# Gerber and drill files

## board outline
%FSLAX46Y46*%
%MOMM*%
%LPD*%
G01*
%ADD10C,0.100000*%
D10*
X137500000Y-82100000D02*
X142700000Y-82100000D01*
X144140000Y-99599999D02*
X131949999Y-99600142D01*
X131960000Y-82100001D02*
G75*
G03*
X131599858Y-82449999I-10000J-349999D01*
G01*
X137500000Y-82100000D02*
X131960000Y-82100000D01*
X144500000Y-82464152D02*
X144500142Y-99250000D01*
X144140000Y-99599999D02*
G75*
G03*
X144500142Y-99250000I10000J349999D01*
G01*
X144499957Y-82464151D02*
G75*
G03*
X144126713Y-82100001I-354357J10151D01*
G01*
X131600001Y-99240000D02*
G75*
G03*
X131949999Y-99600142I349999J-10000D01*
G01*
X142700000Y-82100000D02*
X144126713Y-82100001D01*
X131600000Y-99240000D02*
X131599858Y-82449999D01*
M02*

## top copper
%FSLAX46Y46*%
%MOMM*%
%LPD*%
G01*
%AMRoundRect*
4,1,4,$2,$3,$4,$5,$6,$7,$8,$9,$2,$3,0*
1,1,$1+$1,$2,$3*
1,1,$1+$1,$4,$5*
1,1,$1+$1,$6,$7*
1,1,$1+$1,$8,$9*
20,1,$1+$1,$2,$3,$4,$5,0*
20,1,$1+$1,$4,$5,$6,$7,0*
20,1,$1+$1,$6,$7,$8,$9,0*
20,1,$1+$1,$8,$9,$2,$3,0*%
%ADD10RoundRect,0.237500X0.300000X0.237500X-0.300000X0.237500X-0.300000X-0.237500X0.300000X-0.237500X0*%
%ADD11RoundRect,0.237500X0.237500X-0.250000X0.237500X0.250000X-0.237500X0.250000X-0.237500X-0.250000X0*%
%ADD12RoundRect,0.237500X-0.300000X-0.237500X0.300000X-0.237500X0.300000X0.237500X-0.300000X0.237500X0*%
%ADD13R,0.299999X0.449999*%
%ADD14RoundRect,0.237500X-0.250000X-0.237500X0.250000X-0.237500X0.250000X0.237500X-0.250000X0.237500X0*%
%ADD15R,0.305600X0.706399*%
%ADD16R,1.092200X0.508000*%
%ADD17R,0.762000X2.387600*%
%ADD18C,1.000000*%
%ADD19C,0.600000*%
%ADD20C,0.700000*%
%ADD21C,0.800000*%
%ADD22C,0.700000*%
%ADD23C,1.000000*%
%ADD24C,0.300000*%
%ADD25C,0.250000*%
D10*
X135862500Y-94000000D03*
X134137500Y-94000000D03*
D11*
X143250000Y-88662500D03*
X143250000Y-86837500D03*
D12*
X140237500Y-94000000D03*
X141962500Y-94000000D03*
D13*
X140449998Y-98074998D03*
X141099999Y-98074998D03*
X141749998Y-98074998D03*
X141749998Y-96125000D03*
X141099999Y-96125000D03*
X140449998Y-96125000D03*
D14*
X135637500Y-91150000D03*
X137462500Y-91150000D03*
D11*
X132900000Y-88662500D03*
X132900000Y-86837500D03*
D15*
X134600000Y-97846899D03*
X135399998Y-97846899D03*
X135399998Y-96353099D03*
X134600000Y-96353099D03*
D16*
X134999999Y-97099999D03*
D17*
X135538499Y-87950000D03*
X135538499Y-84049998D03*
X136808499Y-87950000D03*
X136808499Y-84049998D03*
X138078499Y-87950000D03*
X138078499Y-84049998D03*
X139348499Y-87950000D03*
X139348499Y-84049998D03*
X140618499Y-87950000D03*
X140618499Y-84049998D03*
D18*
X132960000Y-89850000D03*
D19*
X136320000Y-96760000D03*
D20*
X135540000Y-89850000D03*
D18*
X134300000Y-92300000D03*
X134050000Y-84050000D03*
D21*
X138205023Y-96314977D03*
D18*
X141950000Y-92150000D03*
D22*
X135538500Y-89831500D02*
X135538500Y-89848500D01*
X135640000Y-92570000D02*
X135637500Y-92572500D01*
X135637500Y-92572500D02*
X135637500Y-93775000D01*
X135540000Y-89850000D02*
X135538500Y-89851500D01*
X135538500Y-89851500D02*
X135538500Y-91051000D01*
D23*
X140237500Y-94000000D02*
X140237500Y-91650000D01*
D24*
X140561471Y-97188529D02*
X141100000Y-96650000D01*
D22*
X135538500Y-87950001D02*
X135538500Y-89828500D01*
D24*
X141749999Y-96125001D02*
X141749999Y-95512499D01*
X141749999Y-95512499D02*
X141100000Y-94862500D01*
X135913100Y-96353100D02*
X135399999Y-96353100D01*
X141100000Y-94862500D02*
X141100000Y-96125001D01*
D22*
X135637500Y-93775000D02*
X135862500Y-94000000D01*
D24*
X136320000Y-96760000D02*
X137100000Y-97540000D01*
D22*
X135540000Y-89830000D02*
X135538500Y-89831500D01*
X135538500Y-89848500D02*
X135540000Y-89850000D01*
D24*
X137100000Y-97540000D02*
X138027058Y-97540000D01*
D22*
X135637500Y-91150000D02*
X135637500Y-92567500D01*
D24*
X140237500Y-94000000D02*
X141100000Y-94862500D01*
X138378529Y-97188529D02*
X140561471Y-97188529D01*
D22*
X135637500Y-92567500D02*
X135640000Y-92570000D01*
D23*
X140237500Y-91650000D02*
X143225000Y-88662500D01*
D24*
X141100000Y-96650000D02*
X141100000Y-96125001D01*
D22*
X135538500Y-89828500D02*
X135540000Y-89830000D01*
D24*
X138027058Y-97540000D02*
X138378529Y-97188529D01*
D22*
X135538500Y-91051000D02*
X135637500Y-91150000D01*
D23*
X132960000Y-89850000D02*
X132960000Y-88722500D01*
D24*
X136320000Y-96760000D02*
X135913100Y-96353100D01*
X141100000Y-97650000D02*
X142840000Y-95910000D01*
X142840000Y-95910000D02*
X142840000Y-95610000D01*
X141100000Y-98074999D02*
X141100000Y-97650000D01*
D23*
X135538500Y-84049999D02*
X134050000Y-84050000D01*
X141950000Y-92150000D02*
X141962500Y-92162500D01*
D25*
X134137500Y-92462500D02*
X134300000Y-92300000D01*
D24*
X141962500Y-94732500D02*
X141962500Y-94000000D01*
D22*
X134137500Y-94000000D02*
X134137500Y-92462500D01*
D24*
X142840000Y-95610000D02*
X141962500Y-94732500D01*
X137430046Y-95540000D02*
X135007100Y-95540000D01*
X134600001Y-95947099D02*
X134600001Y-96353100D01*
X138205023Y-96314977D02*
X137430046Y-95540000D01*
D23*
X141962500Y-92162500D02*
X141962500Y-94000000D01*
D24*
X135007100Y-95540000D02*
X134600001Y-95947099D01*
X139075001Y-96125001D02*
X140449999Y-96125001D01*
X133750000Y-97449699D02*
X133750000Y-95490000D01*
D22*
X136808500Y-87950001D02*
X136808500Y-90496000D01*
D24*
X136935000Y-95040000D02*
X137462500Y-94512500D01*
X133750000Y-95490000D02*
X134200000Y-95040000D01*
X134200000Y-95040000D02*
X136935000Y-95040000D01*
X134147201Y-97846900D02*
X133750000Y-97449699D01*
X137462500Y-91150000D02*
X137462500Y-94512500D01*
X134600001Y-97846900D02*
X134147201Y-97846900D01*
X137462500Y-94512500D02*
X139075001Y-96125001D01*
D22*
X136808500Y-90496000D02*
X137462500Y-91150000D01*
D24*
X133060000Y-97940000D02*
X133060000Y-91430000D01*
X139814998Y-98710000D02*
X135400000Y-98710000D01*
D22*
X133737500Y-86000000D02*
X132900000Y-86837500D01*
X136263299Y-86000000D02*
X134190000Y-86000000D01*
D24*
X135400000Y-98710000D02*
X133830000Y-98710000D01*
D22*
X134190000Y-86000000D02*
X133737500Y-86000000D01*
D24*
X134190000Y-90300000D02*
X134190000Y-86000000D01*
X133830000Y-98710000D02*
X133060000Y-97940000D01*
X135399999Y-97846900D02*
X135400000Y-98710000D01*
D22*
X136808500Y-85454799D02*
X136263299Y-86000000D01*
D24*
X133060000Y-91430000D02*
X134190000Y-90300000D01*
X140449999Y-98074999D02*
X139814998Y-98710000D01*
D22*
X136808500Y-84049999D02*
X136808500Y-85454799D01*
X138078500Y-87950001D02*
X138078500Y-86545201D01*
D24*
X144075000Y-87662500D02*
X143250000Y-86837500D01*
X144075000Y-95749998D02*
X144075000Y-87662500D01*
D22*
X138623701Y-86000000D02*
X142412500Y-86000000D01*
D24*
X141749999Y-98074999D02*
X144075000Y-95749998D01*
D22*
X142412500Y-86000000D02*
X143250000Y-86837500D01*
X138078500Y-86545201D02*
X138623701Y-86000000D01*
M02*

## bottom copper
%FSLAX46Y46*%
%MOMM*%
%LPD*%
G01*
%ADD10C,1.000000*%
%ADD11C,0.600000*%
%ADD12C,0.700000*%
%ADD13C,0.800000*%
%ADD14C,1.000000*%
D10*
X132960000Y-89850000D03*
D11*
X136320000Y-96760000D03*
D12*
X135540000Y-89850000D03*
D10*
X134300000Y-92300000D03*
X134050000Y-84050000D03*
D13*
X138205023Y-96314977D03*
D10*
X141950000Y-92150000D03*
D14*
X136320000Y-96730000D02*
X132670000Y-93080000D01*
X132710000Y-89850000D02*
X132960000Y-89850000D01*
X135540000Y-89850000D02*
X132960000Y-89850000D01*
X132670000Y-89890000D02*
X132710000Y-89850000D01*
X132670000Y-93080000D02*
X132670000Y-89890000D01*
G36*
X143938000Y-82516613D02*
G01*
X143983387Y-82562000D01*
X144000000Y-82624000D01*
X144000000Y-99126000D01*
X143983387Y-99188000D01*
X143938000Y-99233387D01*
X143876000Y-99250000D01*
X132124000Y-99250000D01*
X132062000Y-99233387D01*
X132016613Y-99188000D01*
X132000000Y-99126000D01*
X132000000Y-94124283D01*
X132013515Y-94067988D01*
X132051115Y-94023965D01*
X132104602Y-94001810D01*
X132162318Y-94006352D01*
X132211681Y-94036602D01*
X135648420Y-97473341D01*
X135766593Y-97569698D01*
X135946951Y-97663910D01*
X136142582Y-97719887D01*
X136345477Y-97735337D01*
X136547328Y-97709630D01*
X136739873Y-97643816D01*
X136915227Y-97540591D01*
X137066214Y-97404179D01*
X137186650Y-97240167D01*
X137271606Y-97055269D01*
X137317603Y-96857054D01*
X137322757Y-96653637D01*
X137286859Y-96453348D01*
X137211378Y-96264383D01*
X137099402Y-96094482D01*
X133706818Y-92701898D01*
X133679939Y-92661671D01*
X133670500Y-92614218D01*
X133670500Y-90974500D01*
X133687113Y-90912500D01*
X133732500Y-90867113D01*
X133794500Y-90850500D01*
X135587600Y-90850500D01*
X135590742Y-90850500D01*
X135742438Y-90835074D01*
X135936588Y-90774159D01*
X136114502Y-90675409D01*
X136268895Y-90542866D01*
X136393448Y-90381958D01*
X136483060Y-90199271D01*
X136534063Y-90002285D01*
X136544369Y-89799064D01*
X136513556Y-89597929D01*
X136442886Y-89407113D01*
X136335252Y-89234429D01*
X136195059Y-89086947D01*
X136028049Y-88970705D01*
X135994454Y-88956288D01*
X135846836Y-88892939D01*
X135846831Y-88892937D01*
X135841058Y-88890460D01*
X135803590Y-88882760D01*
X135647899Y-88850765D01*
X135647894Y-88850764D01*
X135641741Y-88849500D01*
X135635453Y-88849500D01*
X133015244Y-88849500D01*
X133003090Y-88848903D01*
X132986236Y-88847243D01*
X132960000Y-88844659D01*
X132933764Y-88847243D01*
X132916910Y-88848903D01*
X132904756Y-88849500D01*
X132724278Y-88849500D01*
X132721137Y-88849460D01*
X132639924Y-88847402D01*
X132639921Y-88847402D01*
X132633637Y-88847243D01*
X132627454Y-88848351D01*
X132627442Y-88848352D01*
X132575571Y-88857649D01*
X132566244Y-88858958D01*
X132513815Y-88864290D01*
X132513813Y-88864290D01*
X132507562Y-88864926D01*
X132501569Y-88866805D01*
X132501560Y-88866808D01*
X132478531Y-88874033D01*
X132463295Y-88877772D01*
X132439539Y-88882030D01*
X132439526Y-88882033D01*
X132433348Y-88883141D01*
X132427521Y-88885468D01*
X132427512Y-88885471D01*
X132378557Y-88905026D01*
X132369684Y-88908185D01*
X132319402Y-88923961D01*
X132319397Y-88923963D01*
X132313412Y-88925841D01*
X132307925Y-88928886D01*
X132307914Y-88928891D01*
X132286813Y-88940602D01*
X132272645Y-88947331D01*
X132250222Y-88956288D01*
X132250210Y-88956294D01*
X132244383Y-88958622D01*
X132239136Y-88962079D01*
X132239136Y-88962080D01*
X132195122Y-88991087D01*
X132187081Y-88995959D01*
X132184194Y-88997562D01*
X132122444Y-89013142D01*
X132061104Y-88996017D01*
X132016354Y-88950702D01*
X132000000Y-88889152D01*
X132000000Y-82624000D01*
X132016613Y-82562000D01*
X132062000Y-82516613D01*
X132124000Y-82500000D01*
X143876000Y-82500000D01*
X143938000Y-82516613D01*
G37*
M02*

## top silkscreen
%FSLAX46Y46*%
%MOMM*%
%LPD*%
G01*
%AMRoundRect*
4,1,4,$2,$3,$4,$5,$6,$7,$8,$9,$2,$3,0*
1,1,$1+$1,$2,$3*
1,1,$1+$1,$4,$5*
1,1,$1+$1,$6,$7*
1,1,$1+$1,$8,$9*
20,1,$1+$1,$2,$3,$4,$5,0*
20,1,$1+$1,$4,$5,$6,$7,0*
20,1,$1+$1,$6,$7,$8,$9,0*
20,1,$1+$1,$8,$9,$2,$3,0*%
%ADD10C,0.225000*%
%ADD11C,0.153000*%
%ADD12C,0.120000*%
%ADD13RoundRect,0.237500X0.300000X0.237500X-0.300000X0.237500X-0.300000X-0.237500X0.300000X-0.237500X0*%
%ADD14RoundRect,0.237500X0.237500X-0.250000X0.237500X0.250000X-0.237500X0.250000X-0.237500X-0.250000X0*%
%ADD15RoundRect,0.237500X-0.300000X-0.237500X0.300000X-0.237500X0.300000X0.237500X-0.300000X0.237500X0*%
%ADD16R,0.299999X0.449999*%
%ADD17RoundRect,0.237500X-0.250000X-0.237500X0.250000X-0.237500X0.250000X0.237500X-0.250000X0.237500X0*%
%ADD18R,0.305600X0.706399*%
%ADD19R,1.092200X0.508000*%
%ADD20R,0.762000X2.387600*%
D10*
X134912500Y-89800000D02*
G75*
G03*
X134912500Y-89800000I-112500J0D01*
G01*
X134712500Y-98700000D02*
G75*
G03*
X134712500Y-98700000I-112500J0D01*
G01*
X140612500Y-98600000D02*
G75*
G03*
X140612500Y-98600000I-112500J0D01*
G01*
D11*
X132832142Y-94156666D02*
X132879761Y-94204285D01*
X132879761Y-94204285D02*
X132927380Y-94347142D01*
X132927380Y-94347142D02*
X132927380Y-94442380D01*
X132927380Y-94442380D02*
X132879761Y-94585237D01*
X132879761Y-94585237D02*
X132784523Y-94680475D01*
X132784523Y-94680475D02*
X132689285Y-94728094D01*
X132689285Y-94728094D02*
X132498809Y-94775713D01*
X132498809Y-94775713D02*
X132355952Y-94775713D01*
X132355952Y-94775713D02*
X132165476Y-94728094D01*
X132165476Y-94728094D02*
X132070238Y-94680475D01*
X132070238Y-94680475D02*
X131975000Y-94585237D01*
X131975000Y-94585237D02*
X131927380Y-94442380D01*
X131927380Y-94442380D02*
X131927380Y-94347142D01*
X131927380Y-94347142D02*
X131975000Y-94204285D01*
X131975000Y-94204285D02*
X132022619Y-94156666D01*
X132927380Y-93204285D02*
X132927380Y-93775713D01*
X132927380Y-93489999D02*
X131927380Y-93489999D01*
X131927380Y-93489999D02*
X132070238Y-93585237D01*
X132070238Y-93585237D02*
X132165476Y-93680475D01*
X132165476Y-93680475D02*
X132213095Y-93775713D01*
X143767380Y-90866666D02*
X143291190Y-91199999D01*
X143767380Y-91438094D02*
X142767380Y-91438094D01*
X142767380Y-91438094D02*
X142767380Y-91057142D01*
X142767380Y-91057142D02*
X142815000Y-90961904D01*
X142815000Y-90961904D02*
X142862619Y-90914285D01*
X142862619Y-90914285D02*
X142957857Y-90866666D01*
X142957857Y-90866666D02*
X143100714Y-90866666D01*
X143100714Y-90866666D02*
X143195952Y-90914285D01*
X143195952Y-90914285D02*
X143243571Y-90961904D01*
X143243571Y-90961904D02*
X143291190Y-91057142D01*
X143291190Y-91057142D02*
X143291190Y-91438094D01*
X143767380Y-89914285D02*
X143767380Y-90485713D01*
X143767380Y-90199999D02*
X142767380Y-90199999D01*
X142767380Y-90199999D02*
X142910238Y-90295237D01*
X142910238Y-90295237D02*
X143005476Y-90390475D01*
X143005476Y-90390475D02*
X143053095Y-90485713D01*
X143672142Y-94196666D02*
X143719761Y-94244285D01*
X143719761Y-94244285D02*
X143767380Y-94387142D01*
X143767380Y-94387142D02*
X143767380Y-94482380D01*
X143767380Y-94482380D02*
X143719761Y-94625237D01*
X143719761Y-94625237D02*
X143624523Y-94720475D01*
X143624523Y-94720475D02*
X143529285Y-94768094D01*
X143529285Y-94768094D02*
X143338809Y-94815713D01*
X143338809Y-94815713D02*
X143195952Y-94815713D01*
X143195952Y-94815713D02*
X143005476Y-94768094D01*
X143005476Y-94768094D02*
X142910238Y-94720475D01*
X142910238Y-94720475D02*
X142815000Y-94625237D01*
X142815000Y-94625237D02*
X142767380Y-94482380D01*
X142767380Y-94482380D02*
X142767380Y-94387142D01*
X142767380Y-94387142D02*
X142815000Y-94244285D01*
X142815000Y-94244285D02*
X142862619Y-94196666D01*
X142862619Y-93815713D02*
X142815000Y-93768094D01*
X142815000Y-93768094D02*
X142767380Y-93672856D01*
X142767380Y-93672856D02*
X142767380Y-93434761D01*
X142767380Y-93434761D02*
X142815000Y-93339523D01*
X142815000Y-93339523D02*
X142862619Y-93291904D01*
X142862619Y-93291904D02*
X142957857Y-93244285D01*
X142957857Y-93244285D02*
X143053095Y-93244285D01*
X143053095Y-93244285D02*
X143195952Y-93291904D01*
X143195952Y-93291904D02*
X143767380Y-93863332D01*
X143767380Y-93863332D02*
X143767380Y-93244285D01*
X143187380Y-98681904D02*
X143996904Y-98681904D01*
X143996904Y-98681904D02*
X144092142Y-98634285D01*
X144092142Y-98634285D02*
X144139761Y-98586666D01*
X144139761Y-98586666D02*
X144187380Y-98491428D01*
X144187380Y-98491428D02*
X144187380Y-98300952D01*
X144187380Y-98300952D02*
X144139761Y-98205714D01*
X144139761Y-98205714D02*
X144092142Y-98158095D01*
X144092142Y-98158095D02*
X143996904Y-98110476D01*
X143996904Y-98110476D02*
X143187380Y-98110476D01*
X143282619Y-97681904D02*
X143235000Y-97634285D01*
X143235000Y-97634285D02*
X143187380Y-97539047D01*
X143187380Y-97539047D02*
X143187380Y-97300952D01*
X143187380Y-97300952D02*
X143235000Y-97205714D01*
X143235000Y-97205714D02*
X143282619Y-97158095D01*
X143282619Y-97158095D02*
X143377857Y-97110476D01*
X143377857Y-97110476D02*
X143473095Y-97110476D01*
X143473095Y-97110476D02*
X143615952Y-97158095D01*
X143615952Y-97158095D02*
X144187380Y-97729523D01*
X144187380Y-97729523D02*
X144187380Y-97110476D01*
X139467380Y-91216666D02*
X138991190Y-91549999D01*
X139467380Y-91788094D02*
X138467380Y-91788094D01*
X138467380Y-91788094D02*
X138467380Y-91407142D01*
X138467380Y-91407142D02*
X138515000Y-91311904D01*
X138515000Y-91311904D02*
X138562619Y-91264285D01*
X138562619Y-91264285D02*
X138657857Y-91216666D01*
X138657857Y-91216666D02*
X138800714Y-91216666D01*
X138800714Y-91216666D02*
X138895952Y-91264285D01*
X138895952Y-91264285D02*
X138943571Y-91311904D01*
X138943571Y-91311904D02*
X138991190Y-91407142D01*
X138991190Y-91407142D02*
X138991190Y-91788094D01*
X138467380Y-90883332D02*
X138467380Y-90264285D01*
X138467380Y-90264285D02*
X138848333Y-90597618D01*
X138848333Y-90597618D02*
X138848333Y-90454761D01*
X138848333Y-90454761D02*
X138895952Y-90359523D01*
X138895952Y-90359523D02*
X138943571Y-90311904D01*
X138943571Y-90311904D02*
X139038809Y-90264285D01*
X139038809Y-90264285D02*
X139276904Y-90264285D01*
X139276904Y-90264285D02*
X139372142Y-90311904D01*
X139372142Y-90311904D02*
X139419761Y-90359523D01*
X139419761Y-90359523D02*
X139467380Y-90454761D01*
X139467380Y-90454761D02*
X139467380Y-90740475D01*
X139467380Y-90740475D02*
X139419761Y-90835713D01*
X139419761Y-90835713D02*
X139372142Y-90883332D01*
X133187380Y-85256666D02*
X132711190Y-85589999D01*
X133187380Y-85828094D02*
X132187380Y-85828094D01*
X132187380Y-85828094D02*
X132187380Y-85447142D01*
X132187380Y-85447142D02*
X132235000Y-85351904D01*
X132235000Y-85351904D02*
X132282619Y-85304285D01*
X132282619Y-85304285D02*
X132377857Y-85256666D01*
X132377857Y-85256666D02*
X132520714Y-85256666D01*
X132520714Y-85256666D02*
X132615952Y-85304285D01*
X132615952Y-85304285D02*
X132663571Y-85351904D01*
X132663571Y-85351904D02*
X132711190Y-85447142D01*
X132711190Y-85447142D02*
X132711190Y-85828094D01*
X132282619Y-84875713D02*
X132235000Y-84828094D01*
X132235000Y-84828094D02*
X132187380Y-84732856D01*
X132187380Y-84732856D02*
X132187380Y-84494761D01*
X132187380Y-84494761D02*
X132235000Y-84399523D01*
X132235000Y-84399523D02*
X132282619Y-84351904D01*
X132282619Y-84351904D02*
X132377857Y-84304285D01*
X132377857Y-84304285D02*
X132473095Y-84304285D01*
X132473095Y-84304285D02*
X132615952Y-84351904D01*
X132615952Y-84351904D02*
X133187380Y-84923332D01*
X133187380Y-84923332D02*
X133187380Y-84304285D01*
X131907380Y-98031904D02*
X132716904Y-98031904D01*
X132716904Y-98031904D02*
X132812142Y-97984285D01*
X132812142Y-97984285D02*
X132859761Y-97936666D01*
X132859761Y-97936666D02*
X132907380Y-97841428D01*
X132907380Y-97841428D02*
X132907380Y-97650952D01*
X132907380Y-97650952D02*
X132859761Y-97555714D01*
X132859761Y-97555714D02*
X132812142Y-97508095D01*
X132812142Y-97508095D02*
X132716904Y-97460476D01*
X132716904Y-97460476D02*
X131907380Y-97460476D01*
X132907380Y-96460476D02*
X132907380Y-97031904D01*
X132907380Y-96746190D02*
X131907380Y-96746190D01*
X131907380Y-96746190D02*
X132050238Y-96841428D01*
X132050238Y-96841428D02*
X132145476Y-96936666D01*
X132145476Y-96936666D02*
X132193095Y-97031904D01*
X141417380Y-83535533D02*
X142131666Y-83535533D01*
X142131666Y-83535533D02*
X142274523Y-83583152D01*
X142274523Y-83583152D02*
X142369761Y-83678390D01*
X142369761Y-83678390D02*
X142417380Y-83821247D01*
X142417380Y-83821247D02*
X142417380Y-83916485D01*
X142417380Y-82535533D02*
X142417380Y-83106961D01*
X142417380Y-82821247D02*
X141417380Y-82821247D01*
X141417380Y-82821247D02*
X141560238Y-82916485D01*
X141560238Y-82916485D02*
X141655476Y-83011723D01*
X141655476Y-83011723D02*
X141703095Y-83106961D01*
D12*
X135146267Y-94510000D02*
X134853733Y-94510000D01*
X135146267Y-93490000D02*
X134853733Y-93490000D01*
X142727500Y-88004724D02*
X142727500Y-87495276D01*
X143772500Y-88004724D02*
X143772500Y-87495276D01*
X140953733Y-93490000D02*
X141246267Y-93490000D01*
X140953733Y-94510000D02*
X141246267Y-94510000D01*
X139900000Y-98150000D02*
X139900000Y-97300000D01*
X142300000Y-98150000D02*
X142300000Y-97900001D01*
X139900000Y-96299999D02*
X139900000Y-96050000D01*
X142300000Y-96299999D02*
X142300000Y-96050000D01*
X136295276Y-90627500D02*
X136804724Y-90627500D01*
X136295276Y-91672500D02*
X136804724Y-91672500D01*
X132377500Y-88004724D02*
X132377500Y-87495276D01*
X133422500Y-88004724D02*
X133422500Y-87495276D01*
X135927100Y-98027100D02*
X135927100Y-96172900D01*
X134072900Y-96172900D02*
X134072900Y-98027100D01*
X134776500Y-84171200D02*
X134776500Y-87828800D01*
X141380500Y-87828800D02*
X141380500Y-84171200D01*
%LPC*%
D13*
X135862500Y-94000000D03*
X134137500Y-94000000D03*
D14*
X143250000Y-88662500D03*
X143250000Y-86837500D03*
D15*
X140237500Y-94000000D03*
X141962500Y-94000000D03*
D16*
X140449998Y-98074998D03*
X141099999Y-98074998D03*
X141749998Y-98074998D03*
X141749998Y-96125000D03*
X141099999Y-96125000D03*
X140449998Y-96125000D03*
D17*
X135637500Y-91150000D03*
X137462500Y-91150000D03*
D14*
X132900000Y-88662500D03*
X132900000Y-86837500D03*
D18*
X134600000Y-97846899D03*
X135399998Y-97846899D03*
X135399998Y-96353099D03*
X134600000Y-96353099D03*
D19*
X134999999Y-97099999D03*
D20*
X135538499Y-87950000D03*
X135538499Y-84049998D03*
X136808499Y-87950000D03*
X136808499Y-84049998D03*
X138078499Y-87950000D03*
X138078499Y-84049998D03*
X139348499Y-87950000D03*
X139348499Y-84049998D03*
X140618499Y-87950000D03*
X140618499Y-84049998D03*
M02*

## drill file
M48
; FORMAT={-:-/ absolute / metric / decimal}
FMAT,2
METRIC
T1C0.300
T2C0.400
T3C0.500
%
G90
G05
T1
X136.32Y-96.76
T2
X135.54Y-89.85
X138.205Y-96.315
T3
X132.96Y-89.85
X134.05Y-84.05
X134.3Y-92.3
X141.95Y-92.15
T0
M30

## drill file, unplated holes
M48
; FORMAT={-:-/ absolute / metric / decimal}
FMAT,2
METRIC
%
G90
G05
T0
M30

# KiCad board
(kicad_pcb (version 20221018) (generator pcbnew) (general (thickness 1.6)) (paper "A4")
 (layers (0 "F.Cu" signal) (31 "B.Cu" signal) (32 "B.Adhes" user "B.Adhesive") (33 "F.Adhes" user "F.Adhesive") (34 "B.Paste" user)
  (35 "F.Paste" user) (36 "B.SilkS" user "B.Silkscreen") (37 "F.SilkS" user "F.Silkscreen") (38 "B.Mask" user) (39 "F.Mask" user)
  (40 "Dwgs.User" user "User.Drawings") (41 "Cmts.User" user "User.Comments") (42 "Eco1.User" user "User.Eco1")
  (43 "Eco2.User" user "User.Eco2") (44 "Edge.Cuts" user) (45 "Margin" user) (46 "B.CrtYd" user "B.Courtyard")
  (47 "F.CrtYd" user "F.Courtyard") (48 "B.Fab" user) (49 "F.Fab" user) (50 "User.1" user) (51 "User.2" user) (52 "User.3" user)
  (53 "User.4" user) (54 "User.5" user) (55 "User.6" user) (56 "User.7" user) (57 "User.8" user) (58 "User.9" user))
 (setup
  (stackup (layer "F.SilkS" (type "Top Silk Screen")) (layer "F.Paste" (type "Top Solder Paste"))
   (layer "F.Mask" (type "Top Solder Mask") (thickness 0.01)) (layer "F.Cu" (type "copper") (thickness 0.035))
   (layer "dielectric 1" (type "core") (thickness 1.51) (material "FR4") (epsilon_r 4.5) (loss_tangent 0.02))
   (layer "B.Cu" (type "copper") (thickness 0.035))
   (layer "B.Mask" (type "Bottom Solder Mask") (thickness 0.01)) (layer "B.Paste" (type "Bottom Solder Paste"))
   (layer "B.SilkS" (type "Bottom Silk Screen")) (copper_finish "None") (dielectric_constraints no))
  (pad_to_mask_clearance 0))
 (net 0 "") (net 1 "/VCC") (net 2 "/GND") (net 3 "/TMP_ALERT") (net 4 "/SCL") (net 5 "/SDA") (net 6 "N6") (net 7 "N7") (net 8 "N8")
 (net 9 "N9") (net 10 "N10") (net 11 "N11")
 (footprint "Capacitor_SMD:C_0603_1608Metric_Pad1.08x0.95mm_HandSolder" (layer "F.Cu") (at 135 94 180)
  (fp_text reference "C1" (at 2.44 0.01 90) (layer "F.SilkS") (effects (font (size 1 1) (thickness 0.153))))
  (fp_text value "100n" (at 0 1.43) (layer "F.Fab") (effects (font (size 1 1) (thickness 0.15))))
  (fp_line (start -0.146267 -0.51) (end 0.146267 -0.51) (stroke (width 0.12) (type solid)) (layer "F.SilkS"))
  (fp_line (start -0.146267 0.51) (end 0.146267 0.51) (stroke (width 0.12) (type solid)) (layer "F.SilkS"))
  (pad "1" smd roundrect (at -0.8625 0 180) (size 1.075 0.95) (layers "F.Cu" "F.Paste" "F.Mask") (roundrect_rratio 0.25) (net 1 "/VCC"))
  (pad "2" smd roundrect (at 0.8625 0 180) (size 1.075 0.95) (layers "F.Cu" "F.Paste" "F.Mask") (roundrect_rratio 0.25) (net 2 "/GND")))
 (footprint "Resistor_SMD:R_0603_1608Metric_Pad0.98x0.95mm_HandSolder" (layer "F.Cu") (at 143.25 87.75 90)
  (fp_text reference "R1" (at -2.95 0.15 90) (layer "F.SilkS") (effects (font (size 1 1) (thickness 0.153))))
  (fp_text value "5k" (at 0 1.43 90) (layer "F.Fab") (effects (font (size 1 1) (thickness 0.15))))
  (fp_line (start -0.254724 -0.5225) (end 0.254724 -0.5225) (stroke (width 0.12) (type solid)) (layer "F.SilkS"))
  (fp_line (start -0.254724 0.5225) (end 0.254724 0.5225) (stroke (width 0.12) (type solid)) (layer "F.SilkS"))
  (pad "1" smd roundrect (at -0.9125 0 90) (size 0.975 0.95) (layers "F.Cu" "F.Paste" "F.Mask") (roundrect_rratio 0.25) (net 1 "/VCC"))
  (pad "2" smd roundrect (at 0.9125 0 90) (size 0.975 0.95) (layers "F.Cu" "F.Paste" "F.Mask") (roundrect_rratio 0.25) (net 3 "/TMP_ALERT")))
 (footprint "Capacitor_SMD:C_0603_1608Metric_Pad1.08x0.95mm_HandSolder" (layer "F.Cu") (at 141.1 94)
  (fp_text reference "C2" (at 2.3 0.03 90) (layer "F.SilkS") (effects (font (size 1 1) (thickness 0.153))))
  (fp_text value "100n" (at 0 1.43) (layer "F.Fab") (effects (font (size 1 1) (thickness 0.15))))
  (fp_line (start -0.146267 -0.51) (end 0.146267 -0.51) (stroke (width 0.12) (type solid)) (layer "F.SilkS"))
  (fp_line (start -0.146267 0.51) (end 0.146267 0.51) (stroke (width 0.12) (type solid)) (layer "F.SilkS"))
  (pad "1" smd roundrect (at -0.8625 0) (size 1.075 0.95) (layers "F.Cu" "F.Paste" "F.Mask") (roundrect_rratio 0.25) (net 1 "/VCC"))
  (pad "2" smd roundrect (at 0.8625 0) (size 1.075 0.95) (layers "F.Cu" "F.Paste" "F.Mask") (roundrect_rratio 0.25) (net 2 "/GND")))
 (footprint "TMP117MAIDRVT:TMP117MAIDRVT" (layer "F.Cu") (at 141.1 97.1 90)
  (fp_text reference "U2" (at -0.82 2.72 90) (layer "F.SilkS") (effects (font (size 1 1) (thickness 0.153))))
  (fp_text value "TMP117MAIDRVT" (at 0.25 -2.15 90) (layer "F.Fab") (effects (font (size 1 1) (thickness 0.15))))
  (fp_line (start -1.05 -1.2) (end -0.2 -1.2) (stroke (width 0.12) (type solid)) (layer "F.SilkS"))
  (fp_line (start -1.05 1.2) (end -0.800001 1.2) (stroke (width 0.12) (type solid)) (layer "F.SilkS"))
  (fp_line (start 0.800001 -1.2) (end 1.05 -1.2) (stroke (width 0.12) (type solid)) (layer "F.SilkS"))
  (fp_line (start 0.800001 1.2) (end 1.05 1.2) (stroke (width 0.12) (type solid)) (layer "F.SilkS"))
  (pad "1" smd rect (at -0.974999 -0.650001 180) (size 0.299999 0.449999) (layers "F.Cu" "F.Paste" "F.Mask") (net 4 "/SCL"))
  (pad "2" smd rect (at -0.974999 0 180) (size 0.299999 0.449999) (layers "F.Cu" "F.Paste" "F.Mask") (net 2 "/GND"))
  (pad "3" smd rect (at -0.974999 0.649999 180) (size 0.299999 0.449999) (layers "F.Cu" "F.Paste" "F.Mask") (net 3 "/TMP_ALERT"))
  (pad "4" smd rect (at 0.974999 0.649999 180) (size 0.299999 0.449999) (layers "F.Cu" "F.Paste" "F.Mask") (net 1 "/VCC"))
  (pad "5" smd rect (at 0.974999 0 180) (size 0.299999 0.449999) (layers "F.Cu" "F.Paste" "F.Mask") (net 1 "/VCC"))
  (pad "6" smd rect (at 0.974999 -0.650001 180) (size 0.299999 0.449999) (layers "F.Cu" "F.Paste" "F.Mask") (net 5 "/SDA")))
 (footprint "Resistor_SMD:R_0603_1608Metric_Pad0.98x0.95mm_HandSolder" (layer "F.Cu") (at 136.55 91.15)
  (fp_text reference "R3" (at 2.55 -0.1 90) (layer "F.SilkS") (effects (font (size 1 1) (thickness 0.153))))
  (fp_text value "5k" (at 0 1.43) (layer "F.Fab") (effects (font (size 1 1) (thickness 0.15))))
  (fp_line (start -0.254724 -0.5225) (end 0.254724 -0.5225) (stroke (width 0.12) (type solid)) (layer "F.SilkS"))
  (fp_line (start -0.254724 0.5225) (end 0.254724 0.5225) (stroke (width 0.12) (type solid)) (layer "F.SilkS"))
  (pad "1" smd roundrect (at -0.9125 0) (size 0.975 0.95) (layers "F.Cu" "F.Paste" "F.Mask") (roundrect_rratio 0.25) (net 1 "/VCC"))
  (pad "2" smd roundrect (at 0.9125 0) (size 0.975 0.95) (layers "F.Cu" "F.Paste" "F.Mask") (roundrect_rratio 0.25) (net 5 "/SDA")))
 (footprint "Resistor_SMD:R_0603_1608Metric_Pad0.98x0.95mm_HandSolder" (layer "F.Cu") (at 132.9 87.75 90)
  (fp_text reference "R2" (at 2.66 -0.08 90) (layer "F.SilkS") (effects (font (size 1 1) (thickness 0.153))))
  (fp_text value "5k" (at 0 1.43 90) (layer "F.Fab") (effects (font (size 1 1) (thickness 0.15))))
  (fp_line (start -0.254724 -0.5225) (end 0.254724 -0.5225) (stroke (width 0.12) (type solid)) (layer "F.SilkS"))
  (fp_line (start -0.254724 0.5225) (end 0.254724 0.5225) (stroke (width 0.12) (type solid)) (layer "F.SilkS"))
  (pad "1" smd roundrect (at -0.9125 0 90) (size 0.975 0.95) (layers "F.Cu" "F.Paste" "F.Mask") (roundrect_rratio 0.25) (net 1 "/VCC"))
  (pad "2" smd roundrect (at 0.9125 0 90) (size 0.975 0.95) (layers "F.Cu" "F.Paste" "F.Mask") (roundrect_rratio 0.25) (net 4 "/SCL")))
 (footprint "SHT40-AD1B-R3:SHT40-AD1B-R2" (layer "F.Cu") (at 135 97.1 90)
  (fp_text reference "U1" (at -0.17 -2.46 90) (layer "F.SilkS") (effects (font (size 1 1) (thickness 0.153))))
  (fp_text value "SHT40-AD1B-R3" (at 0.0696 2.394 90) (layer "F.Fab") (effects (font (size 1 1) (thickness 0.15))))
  (fp_line (start -0.9271 0.9271) (end 0.9271 0.9271) (stroke (width 0.12) (type solid)) (layer "F.SilkS"))
  (fp_line (start 0.9271 -0.9271) (end -0.9271 -0.9271) (stroke (width 0.12) (type solid)) (layer "F.SilkS"))
  (pad "1" smd rect (at -0.7469 -0.399999 90) (size 0.706399 0.3056) (layers "F.Cu" "F.Paste" "F.Mask") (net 5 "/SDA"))
  (pad "2" smd rect (at -0.7469 0.399999 90) (size 0.706399 0.3056) (layers "F.Cu" "F.Paste" "F.Mask") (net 4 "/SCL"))
  (pad "3" smd rect (at 0.7469 0.399999 90) (size 0.706399 0.3056) (layers "F.Cu" "F.Paste" "F.Mask") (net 1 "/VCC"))
  (pad "4" smd rect (at 0.7469 -0.399999 90) (size 0.706399 0.3056) (layers "F.Cu" "F.Paste" "F.Mask") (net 2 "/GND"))
  (pad "5" smd rect (at 0 0 90) (size 0.508 1.0922) (layers "F.Cu" "F.Paste" "F.Mask") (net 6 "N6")))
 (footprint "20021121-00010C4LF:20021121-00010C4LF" (layer "F.Cu") (at 138.0785 86)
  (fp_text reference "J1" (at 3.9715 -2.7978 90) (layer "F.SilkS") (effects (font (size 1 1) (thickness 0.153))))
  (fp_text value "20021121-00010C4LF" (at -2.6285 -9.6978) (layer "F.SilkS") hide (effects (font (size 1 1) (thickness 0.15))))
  (fp_line (start -3.302 -1.8288) (end -3.302 1.8288) (stroke (width 0.12) (type solid)) (layer "F.SilkS"))
  (fp_line (start 3.302 1.8288) (end 3.302 -1.8288) (stroke (width 0.12) (type solid)) (layer "F.SilkS"))
  (pad "1" smd rect (at -2.54 1.950001) (size 0.762 2.3876) (layers "F.Cu" "F.Paste" "F.Mask") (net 1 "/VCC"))
  (pad "2" smd rect (at -2.54 -1.950001) (size 0.762 2.3876) (layers "F.Cu" "F.Paste" "F.Mask") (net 2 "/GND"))
  (pad "3" smd rect (at -1.27 1.950001) (size 0.762 2.3876) (layers "F.Cu" "F.Paste" "F.Mask") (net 5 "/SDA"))
  (pad "4" smd rect (at -1.27 -1.950001) (size 0.762 2.3876) (layers "F.Cu" "F.Paste" "F.Mask") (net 4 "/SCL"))
  (pad "5" smd rect (at 0 1.950001) (size 0.762 2.3876) (layers "F.Cu" "F.Paste" "F.Mask") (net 3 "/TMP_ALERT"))
  (pad "6" smd rect (at 0 -1.950001) (size 0.762 2.3876) (layers "F.Cu" "F.Paste" "F.Mask") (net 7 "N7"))
  (pad "7" smd rect (at 1.27 1.950001) (size 0.762 2.3876) (layers "F.Cu" "F.Paste" "F.Mask") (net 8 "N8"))
  (pad "8" smd rect (at 1.27 -1.950001) (size 0.762 2.3876) (layers "F.Cu" "F.Paste" "F.Mask") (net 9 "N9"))
  (pad "9" smd rect (at 2.54 1.950001) (size 0.762 2.3876) (layers "F.Cu" "F.Paste" "F.Mask") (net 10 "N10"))
  (pad "10" smd rect (at 2.54 -1.950001) (size 0.762 2.3876) (layers "F.Cu" "F.Paste" "F.Mask") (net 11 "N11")))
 (gr_circle (center 134.8 89.8) (end 134.95 89.8) (stroke (width 0.15) (type solid)) (fill solid) (layer "F.SilkS"))
 (gr_circle (center 134.6 98.7) (end 134.75 98.7) (stroke (width 0.15) (type solid)) (fill solid) (layer "F.SilkS"))
 (gr_circle (center 140.5 98.6) (end 140.65 98.6) (stroke (width 0.15) (type solid)) (fill solid) (layer "F.SilkS"))
 (gr_line (start 137.5 82.1) (end 142.7 82.1) (stroke (width 0.1) (type default)) (layer "Edge.Cuts"))
 (gr_line (start 144.14 99.599999) (end 131.949999 99.600142) (stroke (width 0.1) (type default)) (layer "Edge.Cuts"))
 (gr_arc (start 131.599858 82.449999) (mid 131.705973 82.198901) (end 131.96 82.1) (stroke (width 0.1) (type default)) (layer "Edge.Cuts"))
 (gr_line (start 137.5 82.1) (end 131.96 82.1) (stroke (width 0.1) (type default)) (layer "Edge.Cuts"))
 (gr_line (start 144.5 82.464152) (end 144.500142 99.25) (stroke (width 0.1) (type default)) (layer "Edge.Cuts"))
 (gr_arc (start 144.500142 99.25) (mid 144.394027 99.501098) (end 144.14 99.599999) (stroke (width 0.1) (type default)) (layer "Edge.Cuts"))
 (gr_arc (start 144.126713 82.100001) (mid 144.393181 82.20025) (end 144.5 82.464152) (stroke (width 0.1) (type default))
  (layer "Edge.Cuts"))
 (gr_arc (start 131.949999 99.600142) (mid 131.698901 99.494027) (end 131.6 99.24) (stroke (width 0.1) (type default)) (layer "Edge.Cuts"))
 (gr_line (start 142.7 82.1) (end 144.126713 82.100001) (stroke (width 0.1) (type default)) (layer "Edge.Cuts"))
 (gr_line (start 131.6 99.24) (end 131.599858 82.449999) (stroke (width 0.1) (type default)) (layer "Edge.Cuts"))
 (segment (start 135.5385 89.8315) (end 135.5385 89.8485) (width 0.7) (layer "F.Cu") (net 1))
 (segment (start 135.64 92.57) (end 135.6375 92.5725) (width 0.7) (layer "F.Cu") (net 1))
 (segment (start 135.6375 92.5725) (end 135.6375 93.775) (width 0.7) (layer "F.Cu") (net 1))
 (segment (start 135.54 89.85) (end 135.5385 89.8515) (width 0.7) (layer "F.Cu") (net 1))
 (segment (start 135.5385 89.8515) (end 135.5385 91.051) (width 0.7) (layer "F.Cu") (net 1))
 (segment (start 140.2375 94) (end 140.2375 91.65) (width 1) (layer "F.Cu") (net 1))
 (segment (start 140.561471 97.188529) (end 141.1 96.65) (width 0.3) (layer "F.Cu") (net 1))
 (segment (start 135.5385 87.950001) (end 135.5385 89.8285) (width 0.7) (layer "F.Cu") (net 1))
 (segment (start 141.749999 96.125001) (end 141.749999 95.512499) (width 0.3) (layer "F.Cu") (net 1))
 (segment (start 141.749999 95.512499) (end 141.1 94.8625) (width 0.3) (layer "F.Cu") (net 1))
 (segment (start 135.9131 96.3531) (end 135.399999 96.3531) (width 0.3) (layer "F.Cu") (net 1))
 (segment (start 141.1 94.8625) (end 141.1 96.125001) (width 0.3) (layer "F.Cu") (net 1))
 (segment (start 135.6375 93.775) (end 135.8625 94) (width 0.7) (layer "F.Cu") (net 1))
 (segment (start 136.32 96.76) (end 137.1 97.54) (width 0.3) (layer "F.Cu") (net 1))
 (segment (start 135.54 89.83) (end 135.5385 89.8315) (width 0.7) (layer "F.Cu") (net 1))
 (segment (start 135.5385 89.8485) (end 135.54 89.85) (width 0.7) (layer "F.Cu") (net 1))
 (segment (start 137.1 97.54) (end 138.027058 97.54) (width 0.3) (layer "F.Cu") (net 1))
 (segment (start 135.6375 91.15) (end 135.6375 92.5675) (width 0.7) (layer "F.Cu") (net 1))
 (segment (start 140.2375 94) (end 141.1 94.8625) (width 0.3) (layer "F.Cu") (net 1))
 (segment (start 138.378529 97.188529) (end 140.561471 97.188529) (width 0.3) (layer "F.Cu") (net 1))
 (segment (start 135.6375 92.5675) (end 135.64 92.57) (width 0.7) (layer "F.Cu") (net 1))
 (segment (start 140.2375 91.65) (end 143.225 88.6625) (width 1) (layer "F.Cu") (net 1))
 (segment (start 141.1 96.65) (end 141.1 96.125001) (width 0.3) (layer "F.Cu") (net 1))
 (segment (start 135.5385 89.8285) (end 135.54 89.83) (width 0.7) (layer "F.Cu") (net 1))
 (segment (start 138.027058 97.54) (end 138.378529 97.188529) (width 0.3) (layer "F.Cu") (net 1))
 (segment (start 135.5385 91.051) (end 135.6375 91.15) (width 0.7) (layer "F.Cu") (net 1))
 (segment (start 132.96 89.85) (end 132.96 88.7225) (width 1) (layer "F.Cu") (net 1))
 (segment (start 136.32 96.76) (end 135.9131 96.3531) (width 0.3) (layer "F.Cu") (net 1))
 (via (at 132.96 89.85) (size 1) (drill 0.5) (layers "F.Cu" "B.Cu") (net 1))
 (via (at 136.32 96.76) (size 0.6) (drill 0.3) (layers "F.Cu" "B.Cu") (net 1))
 (via (at 135.54 89.85) (size 0.7) (drill 0.4) (layers "F.Cu" "B.Cu") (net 1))
 (segment (start 136.32 96.73) (end 132.67 93.08) (width 1) (layer "B.Cu") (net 1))
 (segment (start 132.71 89.85) (end 132.96 89.85) (width 1) (layer "B.Cu") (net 1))
 (segment (start 135.54 89.85) (end 132.96 89.85) (width 1) (layer "B.Cu") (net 1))
 (segment (start 132.67 89.89) (end 132.71 89.85) (width 1) (layer "B.Cu") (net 1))
 (segment (start 132.67 93.08) (end 132.67 89.89) (width 1) (layer "B.Cu") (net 1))
 (segment (start 141.1 97.65) (end 142.84 95.91) (width 0.3) (layer "F.Cu") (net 2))
 (segment (start 142.84 95.91) (end 142.84 95.61) (width 0.3) (layer "F.Cu") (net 2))
 (segment (start 141.1 98.074999) (end 141.1 97.65) (width 0.3) (layer "F.Cu") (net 2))
 (segment (start 135.5385 84.049999) (end 134.05 84.05) (width 1) (layer "F.Cu") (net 2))
 (segment (start 141.95 92.15) (end 141.9625 92.1625) (width 1) (layer "F.Cu") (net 2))
 (segment (start 134.1375 92.4625) (end 134.3 92.3) (width 0.25) (layer "F.Cu") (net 2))
 (segment (start 141.9625 94.7325) (end 141.9625 94) (width 0.3) (layer "F.Cu") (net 2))
 (segment (start 134.1375 94) (end 134.1375 92.4625) (width 0.7) (layer "F.Cu") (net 2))
 (segment (start 142.84 95.61) (end 141.9625 94.7325) (width 0.3) (layer "F.Cu") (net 2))
 (segment (start 137.430046 95.54) (end 135.0071 95.54) (width 0.3) (layer "F.Cu") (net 2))
 (segment (start 134.600001 95.947099) (end 134.600001 96.3531) (width 0.3) (layer "F.Cu") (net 2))
 (segment (start 138.205023 96.314977) (end 137.430046 95.54) (width 0.3) (layer "F.Cu") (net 2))
 (segment (start 141.9625 92.1625) (end 141.9625 94) (width 1) (layer "F.Cu") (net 2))
 (segment (start 135.0071 95.54) (end 134.600001 95.947099) (width 0.3) (layer "F.Cu") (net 2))
 (via (at 134.3 92.3) (size 1) (drill 0.5) (layers "F.Cu" "B.Cu") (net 2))
 (via (at 134.05 84.05) (size 1) (drill 0.5) (layers "F.Cu" "B.Cu") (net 2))
 (via (at 138.205023 96.314977) (size 0.8) (drill 0.4) (layers "F.Cu" "B.Cu") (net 2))
 (via (at 141.95 92.15) (size 1) (drill 0.5) (layers "F.Cu" "B.Cu") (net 2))
 (segment (start 139.075001 96.125001) (end 140.449999 96.125001) (width 0.3) (layer "F.Cu") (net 5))
 (segment (start 133.75 97.449699) (end 133.75 95.49) (width 0.3) (layer "F.Cu") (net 5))
 (segment (start 136.8085 87.950001) (end 136.8085 90.496) (width 0.7) (layer "F.Cu") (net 5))
 (segment (start 136.935 95.04) (end 137.4625 94.5125) (width 0.3) (layer "F.Cu") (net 5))
 (segment (start 133.75 95.49) (end 134.2 95.04) (width 0.3) (layer "F.Cu") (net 5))
 (segment (start 134.2 95.04) (end 136.935 95.04) (width 0.3) (layer "F.Cu") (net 5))
 (segment (start 134.147201 97.8469) (end 133.75 97.449699) (width 0.3) (layer "F.Cu") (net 5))
 (segment (start 137.4625 91.15) (end 137.4625 94.5125) (width 0.3) (layer "F.Cu") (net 5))
 (segment (start 134.600001 97.8469) (end 134.147201 97.8469) (width 0.3) (layer "F.Cu") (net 5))
 (segment (start 137.4625 94.5125) (end 139.075001 96.125001) (width 0.3) (layer "F.Cu") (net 5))
 (segment (start 136.8085 90.496) (end 137.4625 91.15) (width 0.7) (layer "F.Cu") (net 5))
 (segment (start 133.06 97.94) (end 133.06 91.43) (width 0.3) (layer "F.Cu") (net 4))
 (segment (start 139.814998 98.71) (end 135.4 98.71) (width 0.3) (layer "F.Cu") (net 4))
 (segment (start 133.7375 86) (end 132.9 86.8375) (width 0.7) (layer "F.Cu") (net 4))
 (segment (start 136.263299 86) (end 134.19 86) (width 0.7) (layer "F.Cu") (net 4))
 (segment (start 135.4 98.71) (end 133.83 98.71) (width 0.3) (layer "F.Cu") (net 4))
 (segment (start 134.19 86) (end 133.7375 86) (width 0.7) (layer "F.Cu") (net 4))
 (segment (start 134.19 90.3) (end 134.19 86) (width 0.3) (layer "F.Cu") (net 4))
 (segment (start 133.83 98.71) (end 133.06 97.94) (width 0.3) (layer "F.Cu") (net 4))
 (segment (start 135.399999 97.8469) (end 135.4 98.71) (width 0.3) (layer "F.Cu") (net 4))
 (segment (start 136.8085 85.454799) (end 136.263299 86) (width 0.7) (layer "F.Cu") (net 4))
 (segment (start 133.06 91.43) (end 134.19 90.3) (width 0.3) (layer "F.Cu") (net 4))
 (segment (start 140.449999 98.074999) (end 139.814998 98.71) (width 0.3) (layer "F.Cu") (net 4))
 (segment (start 136.8085 84.049999) (end 136.8085 85.454799) (width 0.7) (layer "F.Cu") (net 4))
 (segment (start 138.0785 87.950001) (end 138.0785 86.545201) (width 0.7) (layer "F.Cu") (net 3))
 (segment (start 144.075 87.6625) (end 143.25 86.8375) (width 0.3) (layer "F.Cu") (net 3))
 (segment (start 144.075 95.749998) (end 144.075 87.6625) (width 0.3) (layer "F.Cu") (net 3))
 (segment (start 138.623701 86) (end 142.4125 86) (width 0.7) (layer "F.Cu") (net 3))
 (segment (start 141.749999 98.074999) (end 144.075 95.749998) (width 0.3) (layer "F.Cu") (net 3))
 (segment (start 142.4125 86) (end 143.25 86.8375) (width 0.7) (layer "F.Cu") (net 3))
 (segment (start 138.0785 86.545201) (end 138.623701 86) (width 0.7) (layer "F.Cu") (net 3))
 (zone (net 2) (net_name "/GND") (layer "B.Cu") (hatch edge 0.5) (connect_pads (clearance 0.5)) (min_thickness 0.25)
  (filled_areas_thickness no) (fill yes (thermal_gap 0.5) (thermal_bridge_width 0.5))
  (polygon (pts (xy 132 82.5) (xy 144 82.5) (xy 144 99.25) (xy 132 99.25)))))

